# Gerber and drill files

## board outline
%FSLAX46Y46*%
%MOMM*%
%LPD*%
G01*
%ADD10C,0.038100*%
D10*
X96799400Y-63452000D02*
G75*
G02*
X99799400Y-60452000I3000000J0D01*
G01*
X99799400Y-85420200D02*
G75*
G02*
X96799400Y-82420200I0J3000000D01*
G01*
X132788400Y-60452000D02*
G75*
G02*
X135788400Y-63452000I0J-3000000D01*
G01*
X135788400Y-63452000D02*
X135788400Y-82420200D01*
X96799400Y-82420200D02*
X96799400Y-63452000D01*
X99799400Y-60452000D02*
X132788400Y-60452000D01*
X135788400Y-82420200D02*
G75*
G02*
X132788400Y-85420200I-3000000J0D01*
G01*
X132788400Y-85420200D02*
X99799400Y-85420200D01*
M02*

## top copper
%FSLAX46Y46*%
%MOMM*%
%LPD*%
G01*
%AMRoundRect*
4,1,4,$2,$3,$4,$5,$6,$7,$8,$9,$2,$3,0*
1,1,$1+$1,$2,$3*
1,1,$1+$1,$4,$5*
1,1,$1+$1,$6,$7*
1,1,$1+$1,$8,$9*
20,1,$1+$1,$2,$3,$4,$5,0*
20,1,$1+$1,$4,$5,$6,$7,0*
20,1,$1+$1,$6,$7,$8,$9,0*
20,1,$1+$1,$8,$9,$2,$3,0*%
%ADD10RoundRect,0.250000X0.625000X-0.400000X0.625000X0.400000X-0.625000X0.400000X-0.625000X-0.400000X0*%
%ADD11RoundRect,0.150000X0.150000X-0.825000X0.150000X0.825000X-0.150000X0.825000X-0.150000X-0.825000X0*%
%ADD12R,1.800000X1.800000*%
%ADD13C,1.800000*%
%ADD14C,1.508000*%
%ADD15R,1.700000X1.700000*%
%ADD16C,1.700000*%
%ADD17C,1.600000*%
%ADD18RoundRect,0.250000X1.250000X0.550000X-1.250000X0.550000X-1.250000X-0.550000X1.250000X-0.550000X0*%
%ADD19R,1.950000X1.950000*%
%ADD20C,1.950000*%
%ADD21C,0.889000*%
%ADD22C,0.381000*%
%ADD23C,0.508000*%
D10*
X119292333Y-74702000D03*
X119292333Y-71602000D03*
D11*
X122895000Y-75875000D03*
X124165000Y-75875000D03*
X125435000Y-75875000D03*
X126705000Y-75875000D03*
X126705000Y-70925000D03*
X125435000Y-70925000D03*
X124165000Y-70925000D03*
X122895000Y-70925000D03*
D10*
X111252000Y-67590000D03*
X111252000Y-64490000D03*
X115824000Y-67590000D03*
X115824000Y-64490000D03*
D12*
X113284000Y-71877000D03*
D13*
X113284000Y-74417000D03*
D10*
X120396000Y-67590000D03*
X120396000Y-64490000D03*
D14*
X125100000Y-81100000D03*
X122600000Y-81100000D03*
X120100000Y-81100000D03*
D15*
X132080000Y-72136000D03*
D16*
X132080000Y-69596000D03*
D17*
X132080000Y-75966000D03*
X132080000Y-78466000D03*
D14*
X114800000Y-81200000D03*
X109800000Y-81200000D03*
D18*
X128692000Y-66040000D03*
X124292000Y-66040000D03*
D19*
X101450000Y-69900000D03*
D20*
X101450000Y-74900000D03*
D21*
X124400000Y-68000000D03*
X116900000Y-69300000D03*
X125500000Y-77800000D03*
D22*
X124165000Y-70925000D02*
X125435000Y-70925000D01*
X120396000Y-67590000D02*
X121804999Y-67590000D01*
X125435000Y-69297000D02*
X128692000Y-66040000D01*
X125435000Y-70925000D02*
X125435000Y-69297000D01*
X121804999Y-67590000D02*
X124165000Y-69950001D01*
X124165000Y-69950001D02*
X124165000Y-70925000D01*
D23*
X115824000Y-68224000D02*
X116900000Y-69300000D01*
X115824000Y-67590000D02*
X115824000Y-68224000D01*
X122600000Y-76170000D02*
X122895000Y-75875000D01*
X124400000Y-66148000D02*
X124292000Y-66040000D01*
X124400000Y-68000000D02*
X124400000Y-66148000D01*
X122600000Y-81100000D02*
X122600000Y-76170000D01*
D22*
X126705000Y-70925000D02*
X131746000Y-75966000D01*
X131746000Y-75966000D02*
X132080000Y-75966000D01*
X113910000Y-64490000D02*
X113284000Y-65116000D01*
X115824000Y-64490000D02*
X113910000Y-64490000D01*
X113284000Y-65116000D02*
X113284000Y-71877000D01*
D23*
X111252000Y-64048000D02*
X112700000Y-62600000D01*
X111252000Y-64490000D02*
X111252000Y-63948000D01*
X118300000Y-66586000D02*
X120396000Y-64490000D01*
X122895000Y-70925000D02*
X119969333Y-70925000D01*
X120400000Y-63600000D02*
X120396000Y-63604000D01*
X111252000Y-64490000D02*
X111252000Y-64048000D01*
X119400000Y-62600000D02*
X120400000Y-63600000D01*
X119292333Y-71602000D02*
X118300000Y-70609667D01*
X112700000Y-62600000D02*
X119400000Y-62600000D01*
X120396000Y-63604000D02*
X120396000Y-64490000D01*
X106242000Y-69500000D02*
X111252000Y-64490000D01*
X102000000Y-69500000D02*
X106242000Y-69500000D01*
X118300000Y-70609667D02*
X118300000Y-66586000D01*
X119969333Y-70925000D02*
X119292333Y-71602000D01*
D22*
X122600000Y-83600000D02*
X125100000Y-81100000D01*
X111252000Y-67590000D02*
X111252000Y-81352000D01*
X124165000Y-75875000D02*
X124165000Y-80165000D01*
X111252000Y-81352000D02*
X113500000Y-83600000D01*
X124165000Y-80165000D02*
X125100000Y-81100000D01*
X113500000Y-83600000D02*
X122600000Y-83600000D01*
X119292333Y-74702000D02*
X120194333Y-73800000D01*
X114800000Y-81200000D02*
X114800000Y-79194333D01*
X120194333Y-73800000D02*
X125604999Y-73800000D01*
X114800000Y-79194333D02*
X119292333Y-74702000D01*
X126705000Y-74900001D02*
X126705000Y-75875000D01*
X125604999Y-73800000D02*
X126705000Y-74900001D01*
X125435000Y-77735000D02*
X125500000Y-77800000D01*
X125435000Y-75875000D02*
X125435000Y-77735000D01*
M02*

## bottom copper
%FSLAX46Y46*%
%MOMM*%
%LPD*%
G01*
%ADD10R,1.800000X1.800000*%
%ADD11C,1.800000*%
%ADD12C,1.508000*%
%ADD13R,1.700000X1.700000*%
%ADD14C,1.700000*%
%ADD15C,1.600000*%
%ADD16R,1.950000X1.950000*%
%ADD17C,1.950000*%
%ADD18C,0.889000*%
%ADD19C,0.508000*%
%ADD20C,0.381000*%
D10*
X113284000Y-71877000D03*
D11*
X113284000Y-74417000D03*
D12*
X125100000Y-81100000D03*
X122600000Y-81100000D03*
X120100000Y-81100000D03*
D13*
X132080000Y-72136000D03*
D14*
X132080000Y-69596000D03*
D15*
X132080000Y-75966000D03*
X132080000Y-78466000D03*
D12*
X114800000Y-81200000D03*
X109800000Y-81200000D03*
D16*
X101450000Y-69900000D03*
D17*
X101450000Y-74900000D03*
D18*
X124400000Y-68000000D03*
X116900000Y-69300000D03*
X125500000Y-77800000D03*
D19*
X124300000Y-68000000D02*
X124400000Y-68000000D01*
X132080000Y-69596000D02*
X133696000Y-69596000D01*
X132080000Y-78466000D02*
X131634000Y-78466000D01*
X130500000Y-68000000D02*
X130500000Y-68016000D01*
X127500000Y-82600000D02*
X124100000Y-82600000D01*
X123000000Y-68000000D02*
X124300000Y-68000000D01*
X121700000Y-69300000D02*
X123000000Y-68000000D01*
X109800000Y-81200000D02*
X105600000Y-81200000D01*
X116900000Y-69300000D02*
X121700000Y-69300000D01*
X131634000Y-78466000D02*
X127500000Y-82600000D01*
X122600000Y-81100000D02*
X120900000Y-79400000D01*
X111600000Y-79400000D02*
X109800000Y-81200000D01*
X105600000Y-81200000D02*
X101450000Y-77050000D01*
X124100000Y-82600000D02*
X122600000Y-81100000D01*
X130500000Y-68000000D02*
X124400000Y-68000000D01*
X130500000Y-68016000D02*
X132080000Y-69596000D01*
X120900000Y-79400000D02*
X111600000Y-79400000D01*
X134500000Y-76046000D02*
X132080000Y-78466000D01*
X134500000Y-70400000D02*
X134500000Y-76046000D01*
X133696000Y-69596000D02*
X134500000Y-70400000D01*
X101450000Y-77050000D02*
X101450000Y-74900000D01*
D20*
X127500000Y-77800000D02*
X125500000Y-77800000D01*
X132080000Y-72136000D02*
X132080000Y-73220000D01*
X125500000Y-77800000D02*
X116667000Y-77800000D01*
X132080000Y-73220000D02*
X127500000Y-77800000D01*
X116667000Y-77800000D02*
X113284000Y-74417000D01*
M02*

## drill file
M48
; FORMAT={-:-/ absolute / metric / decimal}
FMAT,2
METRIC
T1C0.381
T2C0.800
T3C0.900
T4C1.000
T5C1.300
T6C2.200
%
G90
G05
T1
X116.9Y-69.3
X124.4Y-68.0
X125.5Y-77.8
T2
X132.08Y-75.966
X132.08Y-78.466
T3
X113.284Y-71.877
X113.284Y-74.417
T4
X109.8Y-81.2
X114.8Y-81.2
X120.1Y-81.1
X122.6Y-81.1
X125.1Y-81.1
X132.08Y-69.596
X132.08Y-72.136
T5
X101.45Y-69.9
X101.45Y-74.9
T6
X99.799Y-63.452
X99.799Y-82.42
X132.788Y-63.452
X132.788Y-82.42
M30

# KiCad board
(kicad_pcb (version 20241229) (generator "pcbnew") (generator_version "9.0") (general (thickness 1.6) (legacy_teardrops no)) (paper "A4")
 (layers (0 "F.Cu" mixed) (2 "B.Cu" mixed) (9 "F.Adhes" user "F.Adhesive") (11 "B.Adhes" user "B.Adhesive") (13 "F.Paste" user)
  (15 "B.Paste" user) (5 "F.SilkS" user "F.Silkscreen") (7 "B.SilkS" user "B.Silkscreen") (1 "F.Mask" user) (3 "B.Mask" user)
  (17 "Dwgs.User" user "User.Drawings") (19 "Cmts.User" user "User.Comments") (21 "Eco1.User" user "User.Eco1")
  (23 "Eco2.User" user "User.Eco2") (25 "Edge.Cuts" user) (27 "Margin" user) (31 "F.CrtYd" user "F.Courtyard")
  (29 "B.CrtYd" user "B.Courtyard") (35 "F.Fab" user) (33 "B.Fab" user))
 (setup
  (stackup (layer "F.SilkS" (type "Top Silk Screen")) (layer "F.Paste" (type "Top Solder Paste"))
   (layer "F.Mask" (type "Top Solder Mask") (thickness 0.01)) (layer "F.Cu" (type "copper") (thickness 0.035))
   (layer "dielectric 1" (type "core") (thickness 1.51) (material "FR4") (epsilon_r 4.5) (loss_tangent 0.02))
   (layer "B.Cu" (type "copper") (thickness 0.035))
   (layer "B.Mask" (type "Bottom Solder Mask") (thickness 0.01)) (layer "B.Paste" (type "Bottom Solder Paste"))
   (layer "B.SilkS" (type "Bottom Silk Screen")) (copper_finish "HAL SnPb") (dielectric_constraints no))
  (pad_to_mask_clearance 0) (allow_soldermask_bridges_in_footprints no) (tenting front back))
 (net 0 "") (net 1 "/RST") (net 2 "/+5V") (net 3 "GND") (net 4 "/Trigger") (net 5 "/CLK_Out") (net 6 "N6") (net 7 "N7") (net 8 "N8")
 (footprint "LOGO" (layer "F.Cu") (at 105.9 63.1 90)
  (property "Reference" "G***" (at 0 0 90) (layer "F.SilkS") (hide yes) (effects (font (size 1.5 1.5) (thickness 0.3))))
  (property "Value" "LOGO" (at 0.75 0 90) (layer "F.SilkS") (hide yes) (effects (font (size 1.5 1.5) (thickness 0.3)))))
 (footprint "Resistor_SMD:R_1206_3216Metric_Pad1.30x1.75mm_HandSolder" (layer "F.Cu") (at 119.292333 73.152 90)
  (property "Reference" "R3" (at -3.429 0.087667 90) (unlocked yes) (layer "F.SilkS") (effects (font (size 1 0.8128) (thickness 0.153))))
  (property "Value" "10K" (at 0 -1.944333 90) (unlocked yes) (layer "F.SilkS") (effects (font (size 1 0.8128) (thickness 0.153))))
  (pad "1" smd roundrect (at -1.55 0 90) (size 1.3 1.75) (layers "F.Cu" "F.Mask" "F.Paste") (roundrect_rratio 0.192308) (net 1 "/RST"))
  (pad "2" smd roundrect (at 1.55 0 90) (size 1.3 1.75) (layers "F.Cu" "F.Mask" "F.Paste") (roundrect_rratio 0.192308) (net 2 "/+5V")))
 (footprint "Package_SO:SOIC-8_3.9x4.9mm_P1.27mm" (layer "F.Cu") (at 124.8 73.4 90)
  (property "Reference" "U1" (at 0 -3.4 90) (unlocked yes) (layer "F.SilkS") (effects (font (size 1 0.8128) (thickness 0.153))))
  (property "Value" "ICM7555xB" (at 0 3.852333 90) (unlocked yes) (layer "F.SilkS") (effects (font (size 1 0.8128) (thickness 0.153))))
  (pad "1" smd roundrect (at -2.475 -1.905 90) (size 1.95 0.6) (layers "F.Cu" "F.Mask" "F.Paste") (roundrect_rratio 0.25) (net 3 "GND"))
  (pad "2" smd roundrect (at -2.475 -0.635 90) (size 1.95 0.6) (layers "F.Cu" "F.Mask" "F.Paste") (roundrect_rratio 0.25) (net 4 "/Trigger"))
  (pad "3" smd roundrect (at -2.475 0.635 90) (size 1.95 0.6) (layers "F.Cu" "F.Mask" "F.Paste") (roundrect_rratio 0.25) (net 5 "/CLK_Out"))
  (pad "4" smd roundrect (at -2.475 1.905 90) (size 1.95 0.6) (layers "F.Cu" "F.Mask" "F.Paste") (roundrect_rratio 0.25) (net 1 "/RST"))
  (pad "5" smd roundrect (at 2.475 1.905 90) (size 1.95 0.6) (layers "F.Cu" "F.Mask" "F.Paste") (roundrect_rratio 0.25) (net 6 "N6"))
  (pad "6" smd roundrect (at 2.475 0.635 90) (size 1.95 0.6) (layers "F.Cu" "F.Mask" "F.Paste") (roundrect_rratio 0.25) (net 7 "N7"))
  (pad "7" smd roundrect (at 2.475 -0.635 90) (size 1.95 0.6) (layers "F.Cu" "F.Mask" "F.Paste") (roundrect_rratio 0.25) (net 7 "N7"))
  (pad "8" smd roundrect (at 2.475 -1.905 90) (size 1.95 0.6) (layers "F.Cu" "F.Mask" "F.Paste") (roundrect_rratio 0.25) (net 2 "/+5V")))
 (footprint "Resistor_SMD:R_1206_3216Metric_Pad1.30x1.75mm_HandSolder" (layer "F.Cu") (at 111.252 66.04 90)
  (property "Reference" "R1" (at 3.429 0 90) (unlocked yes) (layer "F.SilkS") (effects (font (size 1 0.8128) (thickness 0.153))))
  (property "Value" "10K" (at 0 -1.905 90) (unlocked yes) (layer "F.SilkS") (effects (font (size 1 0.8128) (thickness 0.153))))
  (pad "1" smd roundrect (at -1.55 0 90) (size 1.3 1.75) (layers "F.Cu" "F.Mask" "F.Paste") (roundrect_rratio 0.192308) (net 4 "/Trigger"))
  (pad "2" smd roundrect (at 1.55 0 90) (size 1.3 1.75) (layers "F.Cu" "F.Mask" "F.Paste") (roundrect_rratio 0.192308) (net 2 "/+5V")))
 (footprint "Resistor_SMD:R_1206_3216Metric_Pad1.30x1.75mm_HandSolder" (layer "F.Cu") (at 115.824 66.04 90)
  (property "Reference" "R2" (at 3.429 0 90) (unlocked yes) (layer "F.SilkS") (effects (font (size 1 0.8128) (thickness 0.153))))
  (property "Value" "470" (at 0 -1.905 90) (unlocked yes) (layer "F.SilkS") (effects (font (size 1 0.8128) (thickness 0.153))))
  (pad "1" smd roundrect (at -1.55 0 90) (size 1.3 1.75) (layers "F.Cu" "F.Mask" "F.Paste") (roundrect_rratio 0.192308) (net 3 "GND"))
  (pad "2" smd roundrect (at 1.55 0 90) (size 1.3 1.75) (layers "F.Cu" "F.Mask" "F.Paste") (roundrect_rratio 0.192308) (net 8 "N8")))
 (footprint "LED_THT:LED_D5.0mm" (layer "F.Cu") (at 113.284 71.877 -90)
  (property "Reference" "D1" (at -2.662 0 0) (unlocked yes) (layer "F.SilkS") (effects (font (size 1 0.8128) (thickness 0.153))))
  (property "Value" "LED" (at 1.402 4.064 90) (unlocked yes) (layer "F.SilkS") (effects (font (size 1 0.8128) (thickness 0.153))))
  (pad "1" thru_hole rect (at 0 0 270) (size 1.8 1.8) (drill 0.9) (layers "*.Cu" "*.Mask") (remove_unused_layers no) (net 8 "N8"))
  (pad "2" thru_hole circle (at 2.54 0 270) (size 1.8 1.8) (drill 0.9) (layers "*.Cu" "*.Mask") (remove_unused_layers no) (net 5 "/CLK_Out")))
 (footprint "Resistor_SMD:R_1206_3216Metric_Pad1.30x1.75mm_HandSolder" (layer "F.Cu") (at 120.396 66.04 90)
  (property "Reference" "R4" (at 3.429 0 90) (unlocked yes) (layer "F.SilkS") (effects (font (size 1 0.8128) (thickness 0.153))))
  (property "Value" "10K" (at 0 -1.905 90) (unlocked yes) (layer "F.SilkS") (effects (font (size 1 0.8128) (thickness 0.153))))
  (pad "1" smd roundrect (at -1.55 0 90) (size 1.3 1.75) (layers "F.Cu" "F.Mask" "F.Paste") (roundrect_rratio 0.192308) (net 7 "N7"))
  (pad "2" smd roundrect (at 1.55 0 90) (size 1.3 1.75) (layers "F.Cu" "F.Mask" "F.Paste") (roundrect_rratio 0.192308) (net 2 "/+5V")))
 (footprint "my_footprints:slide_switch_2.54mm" (layer "F.Cu") (at 122.6 81.1 180)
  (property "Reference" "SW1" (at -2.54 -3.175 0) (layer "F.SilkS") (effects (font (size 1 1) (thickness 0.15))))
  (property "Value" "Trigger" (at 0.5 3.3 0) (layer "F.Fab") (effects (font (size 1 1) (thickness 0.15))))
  (pad "1" thru_hole circle (at -2.5 0 180) (size 1.508 1.508) (drill 1) (layers "*.Cu" "*.Mask") (remove_unused_layers no)
   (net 4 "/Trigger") (solder_mask_margin 0.102))
  (pad "2" thru_hole circle (at 0 0 180) (size 1.508 1.508) (drill 1) (layers "*.Cu" "*.Mask") (remove_unused_layers no) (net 3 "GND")
   (solder_mask_margin 0.102))
  (pad "3" thru_hole circle (at 2.5 0 180) (size 1.508 1.508) (drill 1) (layers "*.Cu" "*.Mask") (remove_unused_layers no)
   (solder_mask_margin 0.102)))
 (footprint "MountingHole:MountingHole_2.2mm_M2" (layer "F.Cu") (at 99.7994 63.452)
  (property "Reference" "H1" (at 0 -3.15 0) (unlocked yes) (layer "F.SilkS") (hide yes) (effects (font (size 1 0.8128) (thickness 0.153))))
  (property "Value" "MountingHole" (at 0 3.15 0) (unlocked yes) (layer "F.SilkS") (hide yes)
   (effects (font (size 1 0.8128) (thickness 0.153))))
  (pad "" np_thru_hole circle (at 0 0) (size 2.2 2.2) (drill 2.2) (layers "*.Cu" "*.Mask")))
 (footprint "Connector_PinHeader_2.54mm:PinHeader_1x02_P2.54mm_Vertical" (layer "F.Cu") (at 132.08 72.136 180)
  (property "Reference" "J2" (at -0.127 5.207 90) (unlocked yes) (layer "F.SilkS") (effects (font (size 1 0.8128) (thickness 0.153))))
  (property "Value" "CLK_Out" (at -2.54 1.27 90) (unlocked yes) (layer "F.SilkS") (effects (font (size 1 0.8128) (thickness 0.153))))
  (pad "1" thru_hole rect (at 0 0 180) (size 1.7 1.7) (drill 1) (layers "*.Cu" "*.Mask") (remove_unused_layers no) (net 5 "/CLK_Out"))
  (pad "2" thru_hole circle (at 0 2.54 180) (size 1.7 1.7) (drill 1) (layers "*.Cu" "*.Mask") (remove_unused_layers no) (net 3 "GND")))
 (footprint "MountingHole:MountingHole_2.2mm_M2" (layer "F.Cu") (at 132.7884 82.4202)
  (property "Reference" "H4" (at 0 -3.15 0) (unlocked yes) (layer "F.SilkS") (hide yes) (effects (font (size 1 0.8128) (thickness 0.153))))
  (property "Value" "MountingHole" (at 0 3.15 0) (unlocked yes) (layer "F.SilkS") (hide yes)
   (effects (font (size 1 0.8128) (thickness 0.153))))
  (pad "" np_thru_hole circle (at 0 0) (size 2.2 2.2) (drill 2.2) (layers "*.Cu" "*.Mask")))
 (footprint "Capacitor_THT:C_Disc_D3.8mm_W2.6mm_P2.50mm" (layer "F.Cu") (at 132.08 75.966 -90)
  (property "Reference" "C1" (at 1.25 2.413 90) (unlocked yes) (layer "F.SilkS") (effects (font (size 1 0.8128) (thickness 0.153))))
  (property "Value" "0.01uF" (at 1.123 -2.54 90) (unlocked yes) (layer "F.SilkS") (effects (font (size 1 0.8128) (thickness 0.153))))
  (pad "1" thru_hole circle (at 0 0 270) (size 1.6 1.6) (drill 0.8) (layers "*.Cu" "*.Mask") (remove_unused_layers no) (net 6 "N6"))
  (pad "2" thru_hole circle (at 2.5 0 270) (size 1.6 1.6) (drill 0.8) (layers "*.Cu" "*.Mask") (remove_unused_layers no) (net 3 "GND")))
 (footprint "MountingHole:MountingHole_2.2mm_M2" (layer "F.Cu") (at 132.7884 63.452)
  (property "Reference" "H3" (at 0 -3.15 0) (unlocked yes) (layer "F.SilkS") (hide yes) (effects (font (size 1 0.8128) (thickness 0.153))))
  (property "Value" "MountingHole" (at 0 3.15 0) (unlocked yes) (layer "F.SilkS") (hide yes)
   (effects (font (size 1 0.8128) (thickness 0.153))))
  (pad "" np_thru_hole circle (at 0 0) (size 2.2 2.2) (drill 2.2) (layers "*.Cu" "*.Mask")))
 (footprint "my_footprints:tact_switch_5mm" (layer "F.Cu") (at 112.3 81.2 180)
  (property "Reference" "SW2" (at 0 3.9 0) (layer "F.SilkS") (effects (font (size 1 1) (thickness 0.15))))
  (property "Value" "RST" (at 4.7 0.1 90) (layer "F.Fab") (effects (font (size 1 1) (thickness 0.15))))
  (pad "1" thru_hole circle (at -2.5 0 180) (size 1.508 1.508) (drill 1) (layers "*.Cu" "*.Mask") (remove_unused_layers no) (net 1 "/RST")
   (solder_mask_margin 0.102))
  (pad "2" thru_hole circle (at 2.5 0 180) (size 1.508 1.508) (drill 1) (layers "*.Cu" "*.Mask") (remove_unused_layers no) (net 3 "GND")
   (solder_mask_margin 0.102)))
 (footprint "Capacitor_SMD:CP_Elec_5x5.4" (layer "F.Cu") (at 126.492 66.04 180)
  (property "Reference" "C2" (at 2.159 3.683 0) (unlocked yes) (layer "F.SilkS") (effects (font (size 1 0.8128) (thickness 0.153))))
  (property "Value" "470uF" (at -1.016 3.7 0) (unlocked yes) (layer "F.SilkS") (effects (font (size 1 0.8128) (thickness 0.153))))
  (pad "1" smd roundrect (at -2.2 0 180) (size 3 1.6) (layers "F.Cu" "F.Mask" "F.Paste") (roundrect_rratio 0.15625) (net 7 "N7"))
  (pad "2" smd roundrect (at 2.2 0 180) (size 3 1.6) (layers "F.Cu" "F.Mask" "F.Paste") (roundrect_rratio 0.15625) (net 3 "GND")))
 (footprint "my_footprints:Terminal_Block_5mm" (layer "F.Cu") (at 101.45 72.4 -90)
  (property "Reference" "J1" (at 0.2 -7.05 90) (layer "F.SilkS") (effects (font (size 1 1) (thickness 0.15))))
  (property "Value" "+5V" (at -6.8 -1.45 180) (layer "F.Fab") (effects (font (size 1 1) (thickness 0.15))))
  (pad "1" thru_hole rect (at -2.5 0 270) (size 1.95 1.95) (drill 1.3) (layers "*.Cu" "*.Mask") (remove_unused_layers no) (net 2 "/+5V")
   (solder_mask_margin 0.102))
  (pad "2" thru_hole circle (at 2.5 0 270) (size 1.95 1.95) (drill 1.3) (layers "*.Cu" "*.Mask") (remove_unused_layers no) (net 3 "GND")
   (solder_mask_margin 0.102)))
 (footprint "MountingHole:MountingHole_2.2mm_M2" (layer "F.Cu") (at 99.7994 82.4202)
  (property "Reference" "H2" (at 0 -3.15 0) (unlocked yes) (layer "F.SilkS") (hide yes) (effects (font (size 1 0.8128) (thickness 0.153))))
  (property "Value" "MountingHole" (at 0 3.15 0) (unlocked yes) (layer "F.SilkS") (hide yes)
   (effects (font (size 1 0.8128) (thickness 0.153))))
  (pad "" np_thru_hole circle (at 0 0) (size 2.2 2.2) (drill 2.2) (layers "*.Cu" "*.Mask")))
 (gr_arc (start 96.7994 63.452) (mid 97.67808 61.33068) (end 99.7994 60.452) (stroke (width 0.0381) (type default)) (layer "Edge.Cuts"))
 (gr_arc (start 99.7994 85.4202) (mid 97.67808 84.54152) (end 96.7994 82.4202) (stroke (width 0.0381) (type default)) (layer "Edge.Cuts"))
 (gr_arc (start 132.7884 60.452) (mid 134.90972 61.33068) (end 135.7884 63.452) (stroke (width 0.0381) (type default)) (layer "Edge.Cuts"))
 (gr_line (start 135.7884 63.452) (end 135.7884 82.4202) (stroke (width 0.0381) (type default)) (layer "Edge.Cuts"))
 (gr_line (start 96.7994 82.4202) (end 96.7994 63.452) (stroke (width 0.0381) (type default)) (layer "Edge.Cuts"))
 (gr_line (start 99.7994 60.452) (end 132.7884 60.452) (stroke (width 0.0381) (type default)) (layer "Edge.Cuts"))
 (gr_arc (start 135.7884 82.4202) (mid 134.90972 84.54152) (end 132.7884 85.4202) (stroke (width 0.0381) (type default)) (layer "Edge.Cuts"))
 (gr_line (start 132.7884 85.4202) (end 99.7994 85.4202) (stroke (width 0.0381) (type default)) (layer "Edge.Cuts"))
 (segment (start 124.165 70.925) (end 125.435 70.925) (width 0.381) (layer "F.Cu") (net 7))
 (segment (start 120.396 67.59) (end 121.804999 67.59) (width 0.381) (layer "F.Cu") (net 7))
 (segment (start 125.435 69.297) (end 128.692 66.04) (width 0.381) (layer "F.Cu") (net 7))
 (segment (start 125.435 70.925) (end 125.435 69.297) (width 0.381) (layer "F.Cu") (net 7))
 (segment (start 121.804999 67.59) (end 124.165 69.950001) (width 0.381) (layer "F.Cu") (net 7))
 (segment (start 124.165 69.950001) (end 124.165 70.925) (width 0.381) (layer "F.Cu") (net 7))
 (segment (start 115.824 68.224) (end 116.9 69.3) (width 0.508) (layer "F.Cu") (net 3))
 (segment (start 115.824 67.59) (end 115.824 68.224) (width 0.508) (layer "F.Cu") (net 3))
 (segment (start 122.6 76.17) (end 122.895 75.875) (width 0.508) (layer "F.Cu") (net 3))
 (segment (start 124.4 66.148) (end 124.292 66.04) (width 0.508) (layer "F.Cu") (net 3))
 (segment (start 124.4 68) (end 124.4 66.148) (width 0.508) (layer "F.Cu") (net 3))
 (segment (start 122.6 81.1) (end 122.6 76.17) (width 0.508) (layer "F.Cu") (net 3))
 (via (at 124.4 68) (size 0.889) (drill 0.381) (layers "F.Cu" "B.Cu") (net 3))
 (via (at 116.9 69.3) (size 0.889) (drill 0.381) (layers "F.Cu" "B.Cu") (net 3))
 (segment (start 124.3 68) (end 124.4 68) (width 0.508) (layer "B.Cu") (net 3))
 (segment (start 132.08 69.596) (end 133.696 69.596) (width 0.508) (layer "B.Cu") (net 3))
 (segment (start 132.08 78.466) (end 131.634 78.466) (width 0.508) (layer "B.Cu") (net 3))
 (segment (start 130.5 68) (end 130.5 68.016) (width 0.508) (layer "B.Cu") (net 3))
 (segment (start 127.5 82.6) (end 124.1 82.6) (width 0.508) (layer "B.Cu") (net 3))
 (segment (start 123 68) (end 124.3 68) (width 0.508) (layer "B.Cu") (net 3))
 (segment (start 121.7 69.3) (end 123 68) (width 0.508) (layer "B.Cu") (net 3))
 (segment (start 109.8 81.2) (end 105.6 81.2) (width 0.508) (layer "B.Cu") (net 3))
 (segment (start 116.9 69.3) (end 121.7 69.3) (width 0.508) (layer "B.Cu") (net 3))
 (segment (start 131.634 78.466) (end 127.5 82.6) (width 0.508) (layer "B.Cu") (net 3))
 (segment (start 122.6 81.1) (end 120.9 79.4) (width 0.508) (layer "B.Cu") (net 3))
 (segment (start 111.6 79.4) (end 109.8 81.2) (width 0.508) (layer "B.Cu") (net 3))
 (segment (start 105.6 81.2) (end 101.45 77.05) (width 0.508) (layer "B.Cu") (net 3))
 (segment (start 124.1 82.6) (end 122.6 81.1) (width 0.508) (layer "B.Cu") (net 3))
 (segment (start 130.5 68) (end 124.4 68) (width 0.508) (layer "B.Cu") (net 3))
 (segment (start 130.5 68.016) (end 132.08 69.596) (width 0.508) (layer "B.Cu") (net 3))
 (segment (start 120.9 79.4) (end 111.6 79.4) (width 0.508) (layer "B.Cu") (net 3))
 (segment (start 134.5 76.046) (end 132.08 78.466) (width 0.508) (layer "B.Cu") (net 3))
 (segment (start 134.5 70.4) (end 134.5 76.046) (width 0.508) (layer "B.Cu") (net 3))
 (segment (start 133.696 69.596) (end 134.5 70.4) (width 0.508) (layer "B.Cu") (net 3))
 (segment (start 101.45 77.05) (end 101.45 74.9) (width 0.508) (layer "B.Cu") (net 3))
 (segment (start 126.705 70.925) (end 131.746 75.966) (width 0.381) (layer "F.Cu") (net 6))
 (segment (start 131.746 75.966) (end 132.08 75.966) (width 0.381) (layer "F.Cu") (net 6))
 (segment (start 113.91 64.49) (end 113.284 65.116) (width 0.381) (layer "F.Cu") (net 8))
 (segment (start 115.824 64.49) (end 113.91 64.49) (width 0.381) (layer "F.Cu") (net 8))
 (segment (start 113.284 65.116) (end 113.284 71.877) (width 0.381) (layer "F.Cu") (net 8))
 (segment (start 111.252 64.048) (end 112.7 62.6) (width 0.508) (layer "F.Cu") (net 2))
 (segment (start 111.252 64.49) (end 111.252 63.948) (width 0.508) (layer "F.Cu") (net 2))
 (segment (start 118.3 66.586) (end 120.396 64.49) (width 0.508) (layer "F.Cu") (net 2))
 (segment (start 122.895 70.925) (end 119.969333 70.925) (width 0.508) (layer "F.Cu") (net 2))
 (segment (start 120.4 63.6) (end 120.396 63.604) (width 0.508) (layer "F.Cu") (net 2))
 (segment (start 111.252 64.49) (end 111.252 64.048) (width 0.508) (layer "F.Cu") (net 2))
 (segment (start 119.4 62.6) (end 120.4 63.6) (width 0.508) (layer "F.Cu") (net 2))
 (segment (start 119.292333 71.602) (end 118.3 70.609667) (width 0.508) (layer "F.Cu") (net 2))
 (segment (start 112.7 62.6) (end 119.4 62.6) (width 0.508) (layer "F.Cu") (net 2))
 (segment (start 120.396 63.604) (end 120.396 64.49) (width 0.508) (layer "F.Cu") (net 2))
 (segment (start 106.242 69.5) (end 111.252 64.49) (width 0.508) (layer "F.Cu") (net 2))
 (segment (start 102 69.5) (end 106.242 69.5) (width 0.508) (layer "F.Cu") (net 2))
 (segment (start 118.3 70.609667) (end 118.3 66.586) (width 0.508) (layer "F.Cu") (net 2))
 (segment (start 119.969333 70.925) (end 119.292333 71.602) (width 0.508) (layer "F.Cu") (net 2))
 (segment (start 122.6 83.6) (end 125.1 81.1) (width 0.381) (layer "F.Cu") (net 4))
 (segment (start 111.252 67.59) (end 111.252 81.352) (width 0.381) (layer "F.Cu") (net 4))
 (segment (start 124.165 75.875) (end 124.165 80.165) (width 0.381) (layer "F.Cu") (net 4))
 (segment (start 111.252 81.352) (end 113.5 83.6) (width 0.381) (layer "F.Cu") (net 4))
 (segment (start 124.165 80.165) (end 125.1 81.1) (width 0.381) (layer "F.Cu") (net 4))
 (segment (start 113.5 83.6) (end 122.6 83.6) (width 0.381) (layer "F.Cu") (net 4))
 (segment (start 119.292333 74.702) (end 120.194333 73.8) (width 0.381) (layer "F.Cu") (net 1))
 (segment (start 114.8 81.2) (end 114.8 79.194333) (width 0.381) (layer "F.Cu") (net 1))
 (segment (start 120.194333 73.8) (end 125.604999 73.8) (width 0.381) (layer "F.Cu") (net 1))
 (segment (start 114.8 79.194333) (end 119.292333 74.702) (width 0.381) (layer "F.Cu") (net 1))
 (segment (start 126.705 74.900001) (end 126.705 75.875) (width 0.381) (layer "F.Cu") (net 1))
 (segment (start 125.604999 73.8) (end 126.705 74.900001) (width 0.381) (layer "F.Cu") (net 1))
 (segment (start 125.435 77.735) (end 125.5 77.8) (width 0.381) (layer "F.Cu") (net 5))
 (segment (start 125.435 75.875) (end 125.435 77.735) (width 0.381) (layer "F.Cu") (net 5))
 (via (at 125.5 77.8) (size 0.889) (drill 0.381) (layers "F.Cu" "B.Cu") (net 5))
 (segment (start 127.5 77.8) (end 125.5 77.8) (width 0.381) (layer "B.Cu") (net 5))
 (segment (start 132.08 72.136) (end 132.08 73.22) (width 0.381) (layer "B.Cu") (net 5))
 (segment (start 125.5 77.8) (end 116.667 77.8) (width 0.381) (layer "B.Cu") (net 5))
 (segment (start 132.08 73.22) (end 127.5 77.8) (width 0.381) (layer "B.Cu") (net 5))
 (segment (start 116.667 77.8) (end 113.284 74.417) (width 0.381) (layer "B.Cu") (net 5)))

